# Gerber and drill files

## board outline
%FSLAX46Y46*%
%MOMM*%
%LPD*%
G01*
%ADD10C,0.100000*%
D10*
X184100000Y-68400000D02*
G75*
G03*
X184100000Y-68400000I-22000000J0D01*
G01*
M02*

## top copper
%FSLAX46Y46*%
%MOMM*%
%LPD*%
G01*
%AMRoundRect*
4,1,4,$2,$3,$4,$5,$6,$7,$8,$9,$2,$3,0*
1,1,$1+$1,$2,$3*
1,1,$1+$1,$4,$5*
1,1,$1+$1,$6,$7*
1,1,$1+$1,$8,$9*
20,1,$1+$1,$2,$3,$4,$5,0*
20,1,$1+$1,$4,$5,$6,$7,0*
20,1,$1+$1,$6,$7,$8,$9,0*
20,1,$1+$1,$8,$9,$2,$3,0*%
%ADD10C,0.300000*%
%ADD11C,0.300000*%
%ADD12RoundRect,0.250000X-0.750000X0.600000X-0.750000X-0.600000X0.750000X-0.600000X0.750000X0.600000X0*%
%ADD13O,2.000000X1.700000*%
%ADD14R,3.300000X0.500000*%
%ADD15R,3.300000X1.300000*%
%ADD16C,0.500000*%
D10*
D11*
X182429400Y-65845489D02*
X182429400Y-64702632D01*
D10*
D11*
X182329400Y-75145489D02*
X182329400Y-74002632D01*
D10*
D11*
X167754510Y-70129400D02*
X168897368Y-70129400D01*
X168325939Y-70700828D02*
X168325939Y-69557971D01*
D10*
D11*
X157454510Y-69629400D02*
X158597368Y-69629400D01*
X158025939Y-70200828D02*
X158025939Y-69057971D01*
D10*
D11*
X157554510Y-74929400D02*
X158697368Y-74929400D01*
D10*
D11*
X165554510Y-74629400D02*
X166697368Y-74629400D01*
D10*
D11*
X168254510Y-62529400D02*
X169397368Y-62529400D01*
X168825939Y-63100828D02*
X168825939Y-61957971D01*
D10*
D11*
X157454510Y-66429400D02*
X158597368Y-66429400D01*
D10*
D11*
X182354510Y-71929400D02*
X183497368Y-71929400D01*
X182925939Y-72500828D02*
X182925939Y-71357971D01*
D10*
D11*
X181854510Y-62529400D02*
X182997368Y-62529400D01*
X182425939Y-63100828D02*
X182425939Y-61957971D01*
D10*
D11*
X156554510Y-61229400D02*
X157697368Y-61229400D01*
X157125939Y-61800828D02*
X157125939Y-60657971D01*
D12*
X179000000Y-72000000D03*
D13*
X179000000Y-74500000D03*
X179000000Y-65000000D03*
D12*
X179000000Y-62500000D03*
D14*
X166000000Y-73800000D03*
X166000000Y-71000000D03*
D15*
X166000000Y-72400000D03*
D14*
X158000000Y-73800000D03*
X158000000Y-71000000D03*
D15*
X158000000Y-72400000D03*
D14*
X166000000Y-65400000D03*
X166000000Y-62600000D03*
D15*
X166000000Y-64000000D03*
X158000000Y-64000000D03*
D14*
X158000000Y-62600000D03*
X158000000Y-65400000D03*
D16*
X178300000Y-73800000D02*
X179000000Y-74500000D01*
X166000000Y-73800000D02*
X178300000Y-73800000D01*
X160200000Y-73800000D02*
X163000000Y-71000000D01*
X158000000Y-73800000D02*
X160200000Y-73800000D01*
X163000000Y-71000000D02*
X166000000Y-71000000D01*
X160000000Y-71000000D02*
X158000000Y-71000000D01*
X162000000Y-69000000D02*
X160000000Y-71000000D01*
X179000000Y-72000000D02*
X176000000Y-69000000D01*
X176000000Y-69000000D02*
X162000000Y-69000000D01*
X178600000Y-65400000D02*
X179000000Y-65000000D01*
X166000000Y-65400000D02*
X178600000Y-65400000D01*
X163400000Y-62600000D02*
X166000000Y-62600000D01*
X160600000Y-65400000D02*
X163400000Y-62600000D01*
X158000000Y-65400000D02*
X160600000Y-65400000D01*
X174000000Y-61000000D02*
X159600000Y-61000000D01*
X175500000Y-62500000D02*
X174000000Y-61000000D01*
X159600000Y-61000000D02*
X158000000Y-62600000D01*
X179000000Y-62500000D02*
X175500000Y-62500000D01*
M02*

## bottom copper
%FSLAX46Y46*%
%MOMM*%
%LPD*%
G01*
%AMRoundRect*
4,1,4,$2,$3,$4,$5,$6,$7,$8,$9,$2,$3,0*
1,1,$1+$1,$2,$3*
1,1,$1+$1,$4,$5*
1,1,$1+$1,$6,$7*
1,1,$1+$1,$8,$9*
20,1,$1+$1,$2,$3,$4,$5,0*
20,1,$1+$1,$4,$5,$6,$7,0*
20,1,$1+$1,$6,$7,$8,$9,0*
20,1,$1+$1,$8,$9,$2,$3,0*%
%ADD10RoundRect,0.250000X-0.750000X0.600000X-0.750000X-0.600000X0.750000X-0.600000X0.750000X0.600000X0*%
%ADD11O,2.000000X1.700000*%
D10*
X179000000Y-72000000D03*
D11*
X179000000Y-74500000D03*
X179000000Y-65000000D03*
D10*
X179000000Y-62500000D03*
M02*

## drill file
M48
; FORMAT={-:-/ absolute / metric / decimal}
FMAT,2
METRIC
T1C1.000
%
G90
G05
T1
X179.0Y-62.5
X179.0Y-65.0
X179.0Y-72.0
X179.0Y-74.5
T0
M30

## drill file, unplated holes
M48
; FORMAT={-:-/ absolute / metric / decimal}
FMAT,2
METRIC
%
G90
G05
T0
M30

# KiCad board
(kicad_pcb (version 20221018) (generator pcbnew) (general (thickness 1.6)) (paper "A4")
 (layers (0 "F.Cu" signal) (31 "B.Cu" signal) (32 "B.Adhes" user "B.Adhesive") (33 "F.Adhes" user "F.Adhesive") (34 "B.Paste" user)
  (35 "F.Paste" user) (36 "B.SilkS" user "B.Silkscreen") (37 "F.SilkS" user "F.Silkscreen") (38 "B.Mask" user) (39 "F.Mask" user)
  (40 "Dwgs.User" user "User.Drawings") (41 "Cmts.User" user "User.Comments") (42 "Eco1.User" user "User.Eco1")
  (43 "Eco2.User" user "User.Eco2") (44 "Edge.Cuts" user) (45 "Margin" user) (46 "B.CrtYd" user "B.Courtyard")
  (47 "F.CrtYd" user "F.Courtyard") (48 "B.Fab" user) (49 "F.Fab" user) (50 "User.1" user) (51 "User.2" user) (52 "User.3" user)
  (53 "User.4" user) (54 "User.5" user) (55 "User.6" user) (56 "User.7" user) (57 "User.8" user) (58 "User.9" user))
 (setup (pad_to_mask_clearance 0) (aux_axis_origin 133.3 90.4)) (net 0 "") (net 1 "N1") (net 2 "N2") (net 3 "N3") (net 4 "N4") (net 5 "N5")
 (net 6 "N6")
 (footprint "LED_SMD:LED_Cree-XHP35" (layer "F.Cu") (at 166 72.4 90)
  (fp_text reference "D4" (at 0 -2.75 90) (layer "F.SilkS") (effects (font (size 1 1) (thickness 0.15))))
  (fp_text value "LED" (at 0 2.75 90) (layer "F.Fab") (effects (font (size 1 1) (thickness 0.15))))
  (pad "" smd rect (at 0 -1 90) (size 1.01 0.75) (layers "F.Paste"))
  (pad "" smd rect (at 0 0 90) (size 1.01 0.75) (layers "F.Paste"))
  (pad "" smd rect (at 0 1 90) (size 1.01 0.75) (layers "F.Paste"))
  (pad "1" smd rect (at -1.4 0 90) (size 0.5 3.3) (layers "F.Cu" "F.Paste" "F.Mask") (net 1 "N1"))
  (pad "2" smd rect (at 1.4 0 90) (size 0.5 3.3) (layers "F.Cu" "F.Paste" "F.Mask") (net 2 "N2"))
  (pad "3" smd rect (at 0 0 90) (size 1.3 3.3) (layers "F.Cu" "F.Mask")))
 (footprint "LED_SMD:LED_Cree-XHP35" (layer "F.Cu") (at 166 64 90)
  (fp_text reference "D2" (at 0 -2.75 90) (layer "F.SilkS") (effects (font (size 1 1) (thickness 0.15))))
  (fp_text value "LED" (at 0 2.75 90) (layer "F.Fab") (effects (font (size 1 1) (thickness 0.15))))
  (pad "" smd rect (at 0 -1 90) (size 1.01 0.75) (layers "F.Paste"))
  (pad "" smd rect (at 0 0 90) (size 1.01 0.75) (layers "F.Paste"))
  (pad "" smd rect (at 0 1 90) (size 1.01 0.75) (layers "F.Paste"))
  (pad "1" smd rect (at -1.4 0 90) (size 0.5 3.3) (layers "F.Cu" "F.Paste" "F.Mask") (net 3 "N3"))
  (pad "2" smd rect (at 1.4 0 90) (size 0.5 3.3) (layers "F.Cu" "F.Paste" "F.Mask") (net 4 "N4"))
  (pad "3" smd rect (at 0 0 90) (size 1.3 3.3) (layers "F.Cu" "F.Mask")))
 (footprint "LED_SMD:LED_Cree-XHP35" (layer "F.Cu") (at 158 64 90)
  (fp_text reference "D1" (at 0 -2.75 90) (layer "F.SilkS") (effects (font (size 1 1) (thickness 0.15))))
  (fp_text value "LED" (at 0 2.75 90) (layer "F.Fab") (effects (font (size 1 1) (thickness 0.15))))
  (pad "" smd rect (at 0 -1 90) (size 1.01 0.75) (layers "F.Paste"))
  (pad "" smd rect (at 0 0 90) (size 1.01 0.75) (layers "F.Paste"))
  (pad "" smd rect (at 0 1 90) (size 1.01 0.75) (layers "F.Paste"))
  (pad "1" smd rect (at -1.4 0 90) (size 0.5 3.3) (layers "F.Cu" "F.Paste" "F.Mask") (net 4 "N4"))
  (pad "2" smd rect (at 1.4 0 90) (size 0.5 3.3) (layers "F.Cu" "F.Paste" "F.Mask") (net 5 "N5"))
  (pad "3" smd rect (at 0 0 90) (size 1.3 3.3) (layers "F.Cu" "F.Mask")))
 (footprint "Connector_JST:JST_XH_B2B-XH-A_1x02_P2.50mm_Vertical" (layer "F.Cu") (at 179 62.5 -90)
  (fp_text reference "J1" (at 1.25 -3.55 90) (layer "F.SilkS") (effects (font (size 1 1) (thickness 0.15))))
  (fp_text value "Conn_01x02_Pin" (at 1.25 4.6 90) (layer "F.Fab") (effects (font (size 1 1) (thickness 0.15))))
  (pad "1" thru_hole roundrect (at 0 0 270) (size 1.7 2) (drill 1) (layers "*.Cu" "*.Mask") (roundrect_rratio 0.1470588235) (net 5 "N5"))
  (pad "2" thru_hole oval (at 2.5 0 270) (size 1.7 2) (drill 1) (layers "*.Cu" "*.Mask") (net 3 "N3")))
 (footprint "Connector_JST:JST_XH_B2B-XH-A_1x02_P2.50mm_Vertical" (layer "F.Cu") (at 179 72 -90)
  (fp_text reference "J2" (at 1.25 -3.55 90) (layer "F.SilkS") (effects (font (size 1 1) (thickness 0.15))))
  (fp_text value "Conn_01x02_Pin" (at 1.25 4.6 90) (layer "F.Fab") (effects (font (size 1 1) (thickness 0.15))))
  (pad "1" thru_hole roundrect (at 0 0 270) (size 1.7 2) (drill 1) (layers "*.Cu" "*.Mask") (roundrect_rratio 0.1470588235) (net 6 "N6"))
  (pad "2" thru_hole oval (at 2.5 0 270) (size 1.7 2) (drill 1) (layers "*.Cu" "*.Mask") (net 1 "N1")))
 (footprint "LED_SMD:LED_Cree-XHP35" (layer "F.Cu") (at 158 72.4 90)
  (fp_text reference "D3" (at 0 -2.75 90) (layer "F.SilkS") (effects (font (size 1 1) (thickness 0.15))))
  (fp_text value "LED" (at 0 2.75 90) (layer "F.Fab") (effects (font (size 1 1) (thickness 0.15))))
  (pad "" smd rect (at 0 -1 90) (size 1.01 0.75) (layers "F.Paste"))
  (pad "" smd rect (at 0 0 90) (size 1.01 0.75) (layers "F.Paste"))
  (pad "" smd rect (at 0 1 90) (size 1.01 0.75) (layers "F.Paste"))
  (pad "1" smd rect (at -1.4 0 90) (size 0.5 3.3) (layers "F.Cu" "F.Paste" "F.Mask") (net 2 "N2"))
  (pad "2" smd rect (at 1.4 0 90) (size 0.5 3.3) (layers "F.Cu" "F.Paste" "F.Mask") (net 6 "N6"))
  (pad "3" smd rect (at 0 0 90) (size 1.3 3.3) (layers "F.Cu" "F.Mask")))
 (gr_circle (center 162.1 68.4) (end 184.1 68.4) (stroke (width 0.1) (type default)) (fill none) (layer "Edge.Cuts"))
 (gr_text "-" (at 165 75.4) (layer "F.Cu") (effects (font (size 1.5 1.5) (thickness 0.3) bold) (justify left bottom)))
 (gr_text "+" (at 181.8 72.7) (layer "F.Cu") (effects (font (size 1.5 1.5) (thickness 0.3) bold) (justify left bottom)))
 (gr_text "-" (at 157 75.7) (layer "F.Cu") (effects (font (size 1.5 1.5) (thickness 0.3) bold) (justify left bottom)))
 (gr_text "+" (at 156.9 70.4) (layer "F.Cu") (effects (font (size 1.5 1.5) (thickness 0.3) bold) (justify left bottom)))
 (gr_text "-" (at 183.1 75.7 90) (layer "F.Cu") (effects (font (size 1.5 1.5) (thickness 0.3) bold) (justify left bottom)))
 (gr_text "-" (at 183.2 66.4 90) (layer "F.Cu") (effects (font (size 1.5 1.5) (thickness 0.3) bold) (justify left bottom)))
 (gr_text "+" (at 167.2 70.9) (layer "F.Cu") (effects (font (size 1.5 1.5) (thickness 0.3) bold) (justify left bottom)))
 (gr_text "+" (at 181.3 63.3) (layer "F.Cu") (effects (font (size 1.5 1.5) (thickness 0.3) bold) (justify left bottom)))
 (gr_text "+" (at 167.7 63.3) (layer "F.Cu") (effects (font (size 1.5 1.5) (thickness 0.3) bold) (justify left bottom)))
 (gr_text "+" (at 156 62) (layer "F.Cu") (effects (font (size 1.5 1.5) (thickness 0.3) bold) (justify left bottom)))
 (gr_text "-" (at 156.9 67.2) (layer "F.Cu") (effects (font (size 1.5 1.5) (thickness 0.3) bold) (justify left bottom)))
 (segment (start 163.4 62.6) (end 166 62.6) (width 0.5) (layer "F.Cu") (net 4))
 (segment (start 160.6 65.4) (end 163.4 62.6) (width 0.5) (layer "F.Cu") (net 4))
 (segment (start 158 65.4) (end 160.6 65.4) (width 0.5) (layer "F.Cu") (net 4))
 (segment (start 175.5 62.5) (end 174 61) (width 0.5) (layer "F.Cu") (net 5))
 (segment (start 179 62.5) (end 175.5 62.5) (width 0.5) (layer "F.Cu") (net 5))
 (segment (start 159.6 61) (end 158 62.6) (width 0.5) (layer "F.Cu") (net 5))
 (segment (start 174 61) (end 159.6 61) (width 0.5) (layer "F.Cu") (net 5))
 (segment (start 178.6 65.4) (end 179 65) (width 0.5) (layer "F.Cu") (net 3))
 (segment (start 166 65.4) (end 178.6 65.4) (width 0.5) (layer "F.Cu") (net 3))
 (segment (start 158 73.8) (end 160.2 73.8) (width 0.5) (layer "F.Cu") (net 2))
 (segment (start 163 71) (end 166 71) (width 0.5) (layer "F.Cu") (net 2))
 (segment (start 160.2 73.8) (end 163 71) (width 0.5) (layer "F.Cu") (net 2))
 (segment (start 176 69) (end 162 69) (width 0.5) (layer "F.Cu") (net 6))
 (segment (start 179 72) (end 176 69) (width 0.5) (layer "F.Cu") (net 6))
 (segment (start 162 69) (end 160 71) (width 0.5) (layer "F.Cu") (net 6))
 (segment (start 160 71) (end 158 71) (width 0.5) (layer "F.Cu") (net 6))
 (segment (start 178.3 73.8) (end 179 74.5) (width 0.5) (layer "F.Cu") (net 1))
 (segment (start 166 73.8) (end 178.3 73.8) (width 0.5) (layer "F.Cu") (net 1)))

